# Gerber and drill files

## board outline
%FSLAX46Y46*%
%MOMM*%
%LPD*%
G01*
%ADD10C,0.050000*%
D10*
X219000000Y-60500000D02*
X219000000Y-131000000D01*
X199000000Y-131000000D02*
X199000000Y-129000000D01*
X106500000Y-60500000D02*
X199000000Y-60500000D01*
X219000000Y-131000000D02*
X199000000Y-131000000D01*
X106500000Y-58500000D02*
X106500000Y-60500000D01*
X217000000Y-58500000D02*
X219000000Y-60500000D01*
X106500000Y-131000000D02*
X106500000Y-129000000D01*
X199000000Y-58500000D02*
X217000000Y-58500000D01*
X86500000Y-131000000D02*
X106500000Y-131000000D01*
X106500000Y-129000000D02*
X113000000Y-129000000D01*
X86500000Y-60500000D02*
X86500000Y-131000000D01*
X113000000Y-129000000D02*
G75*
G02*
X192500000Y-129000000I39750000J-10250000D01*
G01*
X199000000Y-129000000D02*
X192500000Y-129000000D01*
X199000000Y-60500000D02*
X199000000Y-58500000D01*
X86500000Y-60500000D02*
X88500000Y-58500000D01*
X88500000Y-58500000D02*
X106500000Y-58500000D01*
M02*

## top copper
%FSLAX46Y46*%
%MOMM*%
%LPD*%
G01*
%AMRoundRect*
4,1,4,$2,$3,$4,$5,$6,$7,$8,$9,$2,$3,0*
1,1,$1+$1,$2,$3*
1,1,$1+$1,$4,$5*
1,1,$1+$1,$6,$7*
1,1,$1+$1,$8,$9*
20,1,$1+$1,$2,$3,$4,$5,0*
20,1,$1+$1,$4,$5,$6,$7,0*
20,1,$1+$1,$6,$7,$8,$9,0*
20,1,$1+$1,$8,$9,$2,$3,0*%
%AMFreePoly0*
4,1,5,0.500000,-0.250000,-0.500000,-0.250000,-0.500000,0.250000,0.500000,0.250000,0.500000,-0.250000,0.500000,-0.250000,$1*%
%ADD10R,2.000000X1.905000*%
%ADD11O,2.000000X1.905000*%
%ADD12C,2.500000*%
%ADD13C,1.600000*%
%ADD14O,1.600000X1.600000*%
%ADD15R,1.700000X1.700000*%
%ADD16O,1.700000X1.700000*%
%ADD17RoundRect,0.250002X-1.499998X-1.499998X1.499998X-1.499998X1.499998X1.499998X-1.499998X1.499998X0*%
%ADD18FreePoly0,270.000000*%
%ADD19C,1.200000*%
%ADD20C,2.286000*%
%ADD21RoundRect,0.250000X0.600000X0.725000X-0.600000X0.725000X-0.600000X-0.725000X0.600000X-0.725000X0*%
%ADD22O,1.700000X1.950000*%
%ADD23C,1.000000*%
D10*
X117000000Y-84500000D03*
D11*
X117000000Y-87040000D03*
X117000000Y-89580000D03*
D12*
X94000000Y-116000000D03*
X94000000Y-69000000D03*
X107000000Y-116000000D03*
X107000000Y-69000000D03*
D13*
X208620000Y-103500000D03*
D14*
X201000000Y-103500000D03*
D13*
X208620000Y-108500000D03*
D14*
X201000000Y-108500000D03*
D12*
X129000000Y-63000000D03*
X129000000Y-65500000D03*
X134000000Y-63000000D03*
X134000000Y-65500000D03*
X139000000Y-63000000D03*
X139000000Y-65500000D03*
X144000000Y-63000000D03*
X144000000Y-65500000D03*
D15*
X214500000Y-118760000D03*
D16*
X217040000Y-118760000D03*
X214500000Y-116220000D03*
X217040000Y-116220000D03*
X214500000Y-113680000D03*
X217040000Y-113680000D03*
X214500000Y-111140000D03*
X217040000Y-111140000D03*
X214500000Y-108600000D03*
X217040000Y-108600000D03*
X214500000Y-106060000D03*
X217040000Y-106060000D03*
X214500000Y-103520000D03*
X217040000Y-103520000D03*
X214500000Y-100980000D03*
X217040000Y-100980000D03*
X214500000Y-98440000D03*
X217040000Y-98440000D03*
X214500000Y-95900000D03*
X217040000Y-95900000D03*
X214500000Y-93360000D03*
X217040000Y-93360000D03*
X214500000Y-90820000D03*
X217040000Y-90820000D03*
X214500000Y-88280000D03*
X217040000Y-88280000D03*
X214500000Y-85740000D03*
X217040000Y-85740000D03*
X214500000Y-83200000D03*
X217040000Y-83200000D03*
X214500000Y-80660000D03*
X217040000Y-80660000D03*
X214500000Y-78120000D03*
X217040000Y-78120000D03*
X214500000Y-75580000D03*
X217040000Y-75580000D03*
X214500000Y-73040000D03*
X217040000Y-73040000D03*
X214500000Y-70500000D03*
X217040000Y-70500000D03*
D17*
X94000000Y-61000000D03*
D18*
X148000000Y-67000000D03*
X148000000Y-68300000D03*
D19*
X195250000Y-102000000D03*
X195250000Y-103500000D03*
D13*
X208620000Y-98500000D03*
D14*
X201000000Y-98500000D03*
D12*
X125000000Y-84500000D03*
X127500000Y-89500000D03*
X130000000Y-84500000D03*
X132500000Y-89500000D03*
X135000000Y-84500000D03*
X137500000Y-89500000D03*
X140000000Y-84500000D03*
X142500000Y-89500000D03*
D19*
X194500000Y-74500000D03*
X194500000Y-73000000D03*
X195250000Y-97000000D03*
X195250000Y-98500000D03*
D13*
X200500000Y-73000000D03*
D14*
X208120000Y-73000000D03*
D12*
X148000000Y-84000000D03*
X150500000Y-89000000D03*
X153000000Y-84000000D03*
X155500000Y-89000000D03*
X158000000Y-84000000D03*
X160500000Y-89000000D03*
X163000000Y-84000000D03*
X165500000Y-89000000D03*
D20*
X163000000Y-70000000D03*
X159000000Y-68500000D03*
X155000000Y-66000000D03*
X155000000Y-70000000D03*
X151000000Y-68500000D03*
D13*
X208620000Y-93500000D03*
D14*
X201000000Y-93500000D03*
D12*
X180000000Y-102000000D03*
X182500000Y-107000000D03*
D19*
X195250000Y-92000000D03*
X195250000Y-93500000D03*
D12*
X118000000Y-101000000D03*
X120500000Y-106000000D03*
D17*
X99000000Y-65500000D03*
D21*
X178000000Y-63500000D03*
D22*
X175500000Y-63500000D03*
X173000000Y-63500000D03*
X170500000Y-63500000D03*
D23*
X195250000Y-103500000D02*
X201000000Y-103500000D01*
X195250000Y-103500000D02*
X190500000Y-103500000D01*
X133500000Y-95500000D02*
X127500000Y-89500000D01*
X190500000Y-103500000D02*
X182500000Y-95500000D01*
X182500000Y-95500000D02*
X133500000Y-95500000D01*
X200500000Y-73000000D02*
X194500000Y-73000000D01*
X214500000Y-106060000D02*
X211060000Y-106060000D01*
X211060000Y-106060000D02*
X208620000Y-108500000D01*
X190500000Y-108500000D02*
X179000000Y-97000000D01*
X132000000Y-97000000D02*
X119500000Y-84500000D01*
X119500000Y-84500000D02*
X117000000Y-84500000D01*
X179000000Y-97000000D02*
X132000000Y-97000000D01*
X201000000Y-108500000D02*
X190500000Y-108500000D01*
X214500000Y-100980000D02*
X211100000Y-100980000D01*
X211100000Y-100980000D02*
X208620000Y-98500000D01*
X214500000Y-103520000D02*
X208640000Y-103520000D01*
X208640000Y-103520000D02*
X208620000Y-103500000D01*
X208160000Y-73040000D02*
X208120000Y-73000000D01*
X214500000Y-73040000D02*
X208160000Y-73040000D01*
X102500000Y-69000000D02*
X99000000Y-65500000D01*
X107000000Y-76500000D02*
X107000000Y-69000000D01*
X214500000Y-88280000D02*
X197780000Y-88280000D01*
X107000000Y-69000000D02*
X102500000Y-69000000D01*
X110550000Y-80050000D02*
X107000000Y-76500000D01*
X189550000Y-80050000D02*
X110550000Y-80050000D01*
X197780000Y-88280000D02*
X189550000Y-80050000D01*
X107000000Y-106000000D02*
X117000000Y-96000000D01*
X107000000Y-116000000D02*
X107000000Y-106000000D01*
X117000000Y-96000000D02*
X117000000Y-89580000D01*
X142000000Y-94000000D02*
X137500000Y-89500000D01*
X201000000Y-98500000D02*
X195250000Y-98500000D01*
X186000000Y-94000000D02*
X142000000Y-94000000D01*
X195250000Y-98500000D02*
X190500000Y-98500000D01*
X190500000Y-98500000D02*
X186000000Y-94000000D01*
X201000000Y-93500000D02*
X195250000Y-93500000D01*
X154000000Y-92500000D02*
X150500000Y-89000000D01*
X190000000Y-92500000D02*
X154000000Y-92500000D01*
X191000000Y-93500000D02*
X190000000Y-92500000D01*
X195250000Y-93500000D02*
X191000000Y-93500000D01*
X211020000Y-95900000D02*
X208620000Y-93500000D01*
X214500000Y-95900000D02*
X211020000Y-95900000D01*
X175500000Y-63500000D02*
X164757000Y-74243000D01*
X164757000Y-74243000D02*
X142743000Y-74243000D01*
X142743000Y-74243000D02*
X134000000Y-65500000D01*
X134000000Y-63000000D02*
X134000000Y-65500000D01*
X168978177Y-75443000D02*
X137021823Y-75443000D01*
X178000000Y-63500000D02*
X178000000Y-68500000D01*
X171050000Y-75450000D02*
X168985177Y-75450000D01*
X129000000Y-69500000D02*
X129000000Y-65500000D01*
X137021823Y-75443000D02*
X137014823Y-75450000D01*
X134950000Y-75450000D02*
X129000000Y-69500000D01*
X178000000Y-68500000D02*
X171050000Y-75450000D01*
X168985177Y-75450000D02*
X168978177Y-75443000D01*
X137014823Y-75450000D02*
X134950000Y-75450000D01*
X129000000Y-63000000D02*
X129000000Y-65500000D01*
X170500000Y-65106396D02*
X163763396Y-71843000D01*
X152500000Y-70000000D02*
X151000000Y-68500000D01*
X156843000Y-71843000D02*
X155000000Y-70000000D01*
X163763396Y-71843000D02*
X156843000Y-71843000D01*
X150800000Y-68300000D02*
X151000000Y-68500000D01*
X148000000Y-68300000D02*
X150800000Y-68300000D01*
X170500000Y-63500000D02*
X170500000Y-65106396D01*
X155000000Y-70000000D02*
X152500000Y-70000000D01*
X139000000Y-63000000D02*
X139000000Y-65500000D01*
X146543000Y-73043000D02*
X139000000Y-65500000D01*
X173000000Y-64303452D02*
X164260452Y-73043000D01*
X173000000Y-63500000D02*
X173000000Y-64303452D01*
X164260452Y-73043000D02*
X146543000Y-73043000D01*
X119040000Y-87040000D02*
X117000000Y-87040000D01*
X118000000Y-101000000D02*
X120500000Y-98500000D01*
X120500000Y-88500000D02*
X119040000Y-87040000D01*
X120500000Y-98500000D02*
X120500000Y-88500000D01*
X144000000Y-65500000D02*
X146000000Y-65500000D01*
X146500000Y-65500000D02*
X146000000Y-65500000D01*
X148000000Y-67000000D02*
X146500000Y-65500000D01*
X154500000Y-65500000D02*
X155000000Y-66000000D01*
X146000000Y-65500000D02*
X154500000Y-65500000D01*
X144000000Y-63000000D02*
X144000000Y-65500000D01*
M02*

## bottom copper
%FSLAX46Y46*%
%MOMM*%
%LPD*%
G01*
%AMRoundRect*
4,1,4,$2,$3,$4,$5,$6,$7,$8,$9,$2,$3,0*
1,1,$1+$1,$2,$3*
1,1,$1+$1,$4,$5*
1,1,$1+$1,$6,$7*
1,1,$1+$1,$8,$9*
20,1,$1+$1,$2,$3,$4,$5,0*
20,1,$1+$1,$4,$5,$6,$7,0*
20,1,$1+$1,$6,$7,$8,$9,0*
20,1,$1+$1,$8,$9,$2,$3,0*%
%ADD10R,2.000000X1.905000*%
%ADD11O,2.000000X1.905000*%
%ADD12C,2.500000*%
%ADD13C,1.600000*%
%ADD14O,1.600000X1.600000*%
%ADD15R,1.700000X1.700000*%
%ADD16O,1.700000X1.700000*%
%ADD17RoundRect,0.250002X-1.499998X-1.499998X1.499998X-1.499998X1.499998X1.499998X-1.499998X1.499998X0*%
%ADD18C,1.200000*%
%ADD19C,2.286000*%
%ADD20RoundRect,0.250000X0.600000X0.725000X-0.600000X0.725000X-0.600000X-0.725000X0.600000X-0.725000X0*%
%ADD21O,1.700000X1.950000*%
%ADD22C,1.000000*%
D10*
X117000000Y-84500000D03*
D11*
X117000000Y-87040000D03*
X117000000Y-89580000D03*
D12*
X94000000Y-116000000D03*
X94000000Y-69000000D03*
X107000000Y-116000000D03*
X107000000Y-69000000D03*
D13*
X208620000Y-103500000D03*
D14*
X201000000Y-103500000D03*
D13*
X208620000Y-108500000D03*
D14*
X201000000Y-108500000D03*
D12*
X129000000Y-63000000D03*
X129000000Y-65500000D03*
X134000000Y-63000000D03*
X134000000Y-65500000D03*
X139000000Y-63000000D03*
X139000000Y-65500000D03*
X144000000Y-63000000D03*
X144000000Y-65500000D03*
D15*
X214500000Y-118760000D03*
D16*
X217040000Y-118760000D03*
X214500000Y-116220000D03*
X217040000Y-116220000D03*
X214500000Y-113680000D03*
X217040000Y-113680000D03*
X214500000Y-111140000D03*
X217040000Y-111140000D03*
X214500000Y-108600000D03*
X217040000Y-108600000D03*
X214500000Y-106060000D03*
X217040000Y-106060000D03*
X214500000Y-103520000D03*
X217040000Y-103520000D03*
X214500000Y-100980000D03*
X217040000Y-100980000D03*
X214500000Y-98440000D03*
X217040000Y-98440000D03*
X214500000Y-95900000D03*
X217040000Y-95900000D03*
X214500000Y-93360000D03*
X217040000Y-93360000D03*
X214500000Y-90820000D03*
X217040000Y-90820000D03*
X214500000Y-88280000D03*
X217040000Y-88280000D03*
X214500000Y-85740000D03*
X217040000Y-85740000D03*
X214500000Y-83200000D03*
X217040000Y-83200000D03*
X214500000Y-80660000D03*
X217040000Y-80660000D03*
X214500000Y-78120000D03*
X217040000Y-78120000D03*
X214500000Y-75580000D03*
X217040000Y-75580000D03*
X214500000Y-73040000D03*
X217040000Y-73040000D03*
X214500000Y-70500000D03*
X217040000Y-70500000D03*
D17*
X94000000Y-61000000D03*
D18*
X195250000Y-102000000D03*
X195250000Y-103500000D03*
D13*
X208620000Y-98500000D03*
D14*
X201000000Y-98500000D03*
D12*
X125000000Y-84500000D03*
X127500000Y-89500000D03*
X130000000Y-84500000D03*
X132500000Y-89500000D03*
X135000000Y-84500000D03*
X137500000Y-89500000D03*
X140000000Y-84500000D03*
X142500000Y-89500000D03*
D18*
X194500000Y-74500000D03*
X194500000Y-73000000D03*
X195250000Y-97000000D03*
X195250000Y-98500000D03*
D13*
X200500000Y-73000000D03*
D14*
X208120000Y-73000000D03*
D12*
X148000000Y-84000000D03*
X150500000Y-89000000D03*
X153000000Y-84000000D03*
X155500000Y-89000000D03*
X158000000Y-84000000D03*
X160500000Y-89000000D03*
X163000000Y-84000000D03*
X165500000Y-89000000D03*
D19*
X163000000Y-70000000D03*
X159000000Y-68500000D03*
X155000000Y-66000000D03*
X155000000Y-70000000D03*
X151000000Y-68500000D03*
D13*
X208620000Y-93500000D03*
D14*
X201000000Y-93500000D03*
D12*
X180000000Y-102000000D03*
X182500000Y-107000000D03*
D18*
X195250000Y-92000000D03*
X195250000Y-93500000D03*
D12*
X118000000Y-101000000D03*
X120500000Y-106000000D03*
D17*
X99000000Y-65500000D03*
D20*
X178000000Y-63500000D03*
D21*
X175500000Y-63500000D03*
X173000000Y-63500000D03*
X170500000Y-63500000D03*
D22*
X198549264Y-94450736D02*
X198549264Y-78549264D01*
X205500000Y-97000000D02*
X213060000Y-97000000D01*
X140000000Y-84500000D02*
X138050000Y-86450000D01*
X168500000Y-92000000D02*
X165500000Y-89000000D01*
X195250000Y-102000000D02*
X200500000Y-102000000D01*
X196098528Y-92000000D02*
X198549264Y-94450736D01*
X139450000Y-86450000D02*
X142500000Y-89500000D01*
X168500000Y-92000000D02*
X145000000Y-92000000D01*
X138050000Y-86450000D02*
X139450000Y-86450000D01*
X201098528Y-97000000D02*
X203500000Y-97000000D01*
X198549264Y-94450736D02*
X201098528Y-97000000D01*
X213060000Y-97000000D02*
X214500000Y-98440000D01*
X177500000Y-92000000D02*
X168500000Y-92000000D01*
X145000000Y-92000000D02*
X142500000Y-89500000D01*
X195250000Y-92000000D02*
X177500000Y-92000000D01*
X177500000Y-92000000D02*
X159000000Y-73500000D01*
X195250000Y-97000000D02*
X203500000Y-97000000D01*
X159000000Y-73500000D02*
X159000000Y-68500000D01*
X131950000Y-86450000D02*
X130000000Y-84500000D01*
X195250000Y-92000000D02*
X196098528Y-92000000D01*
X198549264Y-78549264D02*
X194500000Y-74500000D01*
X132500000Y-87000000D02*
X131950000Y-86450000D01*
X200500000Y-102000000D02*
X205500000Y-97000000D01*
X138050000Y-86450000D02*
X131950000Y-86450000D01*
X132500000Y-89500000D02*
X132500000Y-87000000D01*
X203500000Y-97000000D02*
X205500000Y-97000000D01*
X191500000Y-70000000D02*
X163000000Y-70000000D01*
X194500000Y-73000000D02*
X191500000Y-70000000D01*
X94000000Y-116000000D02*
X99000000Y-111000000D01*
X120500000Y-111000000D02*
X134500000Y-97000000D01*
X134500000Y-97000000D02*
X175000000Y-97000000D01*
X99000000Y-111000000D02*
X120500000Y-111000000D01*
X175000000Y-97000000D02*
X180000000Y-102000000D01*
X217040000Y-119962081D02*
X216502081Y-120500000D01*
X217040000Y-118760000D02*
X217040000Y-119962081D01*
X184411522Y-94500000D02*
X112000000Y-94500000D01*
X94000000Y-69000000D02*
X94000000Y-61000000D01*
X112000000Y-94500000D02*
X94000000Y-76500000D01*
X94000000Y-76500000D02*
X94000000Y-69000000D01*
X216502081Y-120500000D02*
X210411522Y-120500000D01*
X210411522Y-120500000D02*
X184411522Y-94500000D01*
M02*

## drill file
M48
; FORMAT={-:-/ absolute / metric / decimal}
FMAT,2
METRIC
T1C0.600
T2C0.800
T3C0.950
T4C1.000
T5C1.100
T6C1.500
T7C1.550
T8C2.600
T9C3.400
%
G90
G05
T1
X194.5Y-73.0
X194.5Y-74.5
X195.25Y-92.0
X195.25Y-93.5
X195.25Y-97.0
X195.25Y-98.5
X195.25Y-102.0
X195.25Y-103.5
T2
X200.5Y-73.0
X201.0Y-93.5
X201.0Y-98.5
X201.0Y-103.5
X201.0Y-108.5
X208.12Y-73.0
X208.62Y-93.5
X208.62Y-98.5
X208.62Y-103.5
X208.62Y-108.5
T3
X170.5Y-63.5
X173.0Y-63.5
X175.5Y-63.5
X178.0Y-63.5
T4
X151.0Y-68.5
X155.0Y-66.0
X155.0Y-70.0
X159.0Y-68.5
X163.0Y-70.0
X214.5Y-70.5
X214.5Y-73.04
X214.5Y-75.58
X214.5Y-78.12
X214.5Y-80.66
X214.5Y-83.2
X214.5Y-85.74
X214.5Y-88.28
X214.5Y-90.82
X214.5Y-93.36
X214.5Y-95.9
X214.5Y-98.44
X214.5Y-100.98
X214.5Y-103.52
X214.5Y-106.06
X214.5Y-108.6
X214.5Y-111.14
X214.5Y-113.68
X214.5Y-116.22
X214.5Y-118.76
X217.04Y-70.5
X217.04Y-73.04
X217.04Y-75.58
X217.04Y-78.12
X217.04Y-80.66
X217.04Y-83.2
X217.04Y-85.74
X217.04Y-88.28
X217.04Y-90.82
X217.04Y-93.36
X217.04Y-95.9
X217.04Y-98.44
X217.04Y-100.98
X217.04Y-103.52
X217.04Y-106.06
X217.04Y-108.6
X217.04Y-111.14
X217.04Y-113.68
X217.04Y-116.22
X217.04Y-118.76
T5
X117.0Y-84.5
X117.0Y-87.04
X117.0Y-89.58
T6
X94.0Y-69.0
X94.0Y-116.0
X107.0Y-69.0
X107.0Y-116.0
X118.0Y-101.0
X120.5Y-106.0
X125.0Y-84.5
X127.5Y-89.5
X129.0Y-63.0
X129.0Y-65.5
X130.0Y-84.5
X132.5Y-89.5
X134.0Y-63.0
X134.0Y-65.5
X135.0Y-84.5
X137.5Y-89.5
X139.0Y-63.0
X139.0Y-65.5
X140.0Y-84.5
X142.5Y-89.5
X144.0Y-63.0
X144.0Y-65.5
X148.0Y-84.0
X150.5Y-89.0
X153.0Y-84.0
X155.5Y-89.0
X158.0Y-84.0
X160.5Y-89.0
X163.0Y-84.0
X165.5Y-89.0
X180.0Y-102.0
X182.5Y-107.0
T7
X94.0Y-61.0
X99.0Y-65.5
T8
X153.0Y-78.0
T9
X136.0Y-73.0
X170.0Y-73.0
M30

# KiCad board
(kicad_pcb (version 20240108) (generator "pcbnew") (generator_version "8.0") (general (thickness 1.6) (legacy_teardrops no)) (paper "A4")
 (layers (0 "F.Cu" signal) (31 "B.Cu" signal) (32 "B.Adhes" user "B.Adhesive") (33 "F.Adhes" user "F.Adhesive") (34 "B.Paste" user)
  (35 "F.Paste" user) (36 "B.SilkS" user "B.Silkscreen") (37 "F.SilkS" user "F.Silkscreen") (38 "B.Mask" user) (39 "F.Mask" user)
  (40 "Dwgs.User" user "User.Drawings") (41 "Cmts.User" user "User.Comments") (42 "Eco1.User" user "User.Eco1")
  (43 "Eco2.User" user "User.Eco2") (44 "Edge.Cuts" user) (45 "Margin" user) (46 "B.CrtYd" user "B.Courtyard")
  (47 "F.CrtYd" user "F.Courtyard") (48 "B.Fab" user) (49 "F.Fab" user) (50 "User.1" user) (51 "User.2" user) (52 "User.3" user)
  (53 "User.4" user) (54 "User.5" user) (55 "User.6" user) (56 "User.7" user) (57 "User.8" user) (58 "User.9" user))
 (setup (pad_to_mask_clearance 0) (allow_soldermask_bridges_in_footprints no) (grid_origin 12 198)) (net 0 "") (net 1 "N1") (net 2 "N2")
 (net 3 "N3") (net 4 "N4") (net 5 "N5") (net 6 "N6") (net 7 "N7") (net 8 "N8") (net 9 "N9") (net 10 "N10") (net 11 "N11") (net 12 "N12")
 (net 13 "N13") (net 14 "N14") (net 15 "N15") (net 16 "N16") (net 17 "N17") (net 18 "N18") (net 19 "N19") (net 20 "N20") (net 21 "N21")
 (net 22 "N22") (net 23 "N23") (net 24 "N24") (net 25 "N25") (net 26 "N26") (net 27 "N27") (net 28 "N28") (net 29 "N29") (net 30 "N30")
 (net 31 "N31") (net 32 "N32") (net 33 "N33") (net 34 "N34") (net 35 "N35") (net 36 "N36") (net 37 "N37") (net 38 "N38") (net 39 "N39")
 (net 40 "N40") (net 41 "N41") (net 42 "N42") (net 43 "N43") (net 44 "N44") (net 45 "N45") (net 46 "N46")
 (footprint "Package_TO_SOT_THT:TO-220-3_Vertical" (layer "F.Cu") (at 117 84.5 -90)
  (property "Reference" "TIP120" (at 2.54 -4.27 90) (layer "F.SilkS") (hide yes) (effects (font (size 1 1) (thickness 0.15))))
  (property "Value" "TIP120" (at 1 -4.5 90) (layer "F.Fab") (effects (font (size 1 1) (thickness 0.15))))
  (pad "1" thru_hole rect (at 0 0 270) (size 1.905 2) (drill 1.1) (layers "*.Cu" "*.Mask") (remove_unused_layers no) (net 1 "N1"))
  (pad "2" thru_hole oval (at 2.54 0 270) (size 1.905 2) (drill 1.1) (layers "*.Cu" "*.Mask") (remove_unused_layers no) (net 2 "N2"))
  (pad "3" thru_hole oval (at 5.08 0 270) (size 1.905 2) (drill 1.1) (layers "*.Cu" "*.Mask") (remove_unused_layers no) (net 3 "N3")))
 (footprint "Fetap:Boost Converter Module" (layer "F.Cu") (at 100.5 117.5)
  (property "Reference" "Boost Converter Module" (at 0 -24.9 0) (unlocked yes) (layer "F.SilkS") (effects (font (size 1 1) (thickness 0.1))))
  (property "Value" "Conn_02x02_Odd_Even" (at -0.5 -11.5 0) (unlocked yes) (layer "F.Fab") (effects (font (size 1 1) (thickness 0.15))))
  (pad "1" thru_hole circle (at -6.5 -1.5) (size 2.5 2.5) (drill 1.5) (layers "*.Cu" "*.Mask") (remove_unused_layers no) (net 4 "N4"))
  (pad "2" thru_hole circle (at -6.5 -48.5) (size 2.5 2.5) (drill 1.5) (layers "*.Cu" "*.Mask") (remove_unused_layers no) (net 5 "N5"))
  (pad "3" thru_hole circle (at 6.5 -1.5) (size 2.5 2.5) (drill 1.5) (layers "*.Cu" "*.Mask") (remove_unused_layers no) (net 3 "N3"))
  (pad "4" thru_hole circle (at 6.5 -48.5) (size 2.5 2.5) (drill 1.5) (layers "*.Cu" "*.Mask") (remove_unused_layers no) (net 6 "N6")))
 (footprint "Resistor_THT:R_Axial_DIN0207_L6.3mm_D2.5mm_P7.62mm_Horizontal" (layer "F.Cu") (at 208.62 103.5 180)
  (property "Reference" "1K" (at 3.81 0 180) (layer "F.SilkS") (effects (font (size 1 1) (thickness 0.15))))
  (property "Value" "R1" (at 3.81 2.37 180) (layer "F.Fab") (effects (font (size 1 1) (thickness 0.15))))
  (pad "1" thru_hole circle (at 0 0 180) (size 1.6 1.6) (drill 0.8) (layers "*.Cu" "*.Mask") (remove_unused_layers no) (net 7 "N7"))
  (pad "2" thru_hole oval (at 7.62 0 180) (size 1.6 1.6) (drill 0.8) (layers "*.Cu" "*.Mask") (remove_unused_layers no) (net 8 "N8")))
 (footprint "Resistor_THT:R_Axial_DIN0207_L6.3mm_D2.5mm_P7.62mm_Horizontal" (layer "F.Cu") (at 208.62 108.5 180)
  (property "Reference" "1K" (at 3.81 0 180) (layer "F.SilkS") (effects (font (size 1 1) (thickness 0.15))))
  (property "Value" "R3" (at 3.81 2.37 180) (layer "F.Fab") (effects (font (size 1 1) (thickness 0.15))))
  (pad "1" thru_hole circle (at 0 0 180) (size 1.6 1.6) (drill 0.8) (layers "*.Cu" "*.Mask") (remove_unused_layers no) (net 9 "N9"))
  (pad "2" thru_hole oval (at 7.62 0 180) (size 1.6 1.6) (drill 0.8) (layers "*.Cu" "*.Mask") (remove_unused_layers no) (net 1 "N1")))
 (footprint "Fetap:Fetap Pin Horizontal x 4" (layer "F.Cu") (at 129 65.5)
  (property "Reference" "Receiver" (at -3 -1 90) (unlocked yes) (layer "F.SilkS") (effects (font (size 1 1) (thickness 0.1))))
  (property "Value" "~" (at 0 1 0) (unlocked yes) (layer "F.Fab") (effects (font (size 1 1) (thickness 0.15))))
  (pad "1" thru_hole circle (at 0 -2.5) (size 2.5 2.5) (drill 1.5) (layers "*.Cu" "*.Mask") (remove_unused_layers no) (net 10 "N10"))
  (pad "1" thru_hole circle (at 0 0) (size 2.5 2.5) (drill 1.5) (layers "*.Cu" "*.Mask") (remove_unused_layers no) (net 10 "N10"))
  (pad "2" thru_hole circle (at 5 -2.5) (size 2.5 2.5) (drill 1.5) (layers "*.Cu" "*.Mask") (remove_unused_layers no) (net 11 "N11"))
  (pad "2" thru_hole circle (at 5 0) (size 2.5 2.5) (drill 1.5) (layers "*.Cu" "*.Mask") (remove_unused_layers no) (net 11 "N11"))
  (pad "3" thru_hole circle (at 10 -2.5) (size 2.5 2.5) (drill 1.5) (layers "*.Cu" "*.Mask") (remove_unused_layers no) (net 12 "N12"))
  (pad "3" thru_hole circle (at 10 0) (size 2.5 2.5) (drill 1.5) (layers "*.Cu" "*.Mask") (remove_unused_layers no) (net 12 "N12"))
  (pad "4" thru_hole circle (at 15 -2.5) (size 2.5 2.5) (drill 1.5) (layers "*.Cu" "*.Mask") (remove_unused_layers no) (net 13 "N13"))
  (pad "4" thru_hole circle (at 15 0) (size 2.5 2.5) (drill 1.5) (layers "*.Cu" "*.Mask") (remove_unused_layers no) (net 13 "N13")))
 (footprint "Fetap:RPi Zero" (layer "F.Cu") (at 214.5 118.76 180)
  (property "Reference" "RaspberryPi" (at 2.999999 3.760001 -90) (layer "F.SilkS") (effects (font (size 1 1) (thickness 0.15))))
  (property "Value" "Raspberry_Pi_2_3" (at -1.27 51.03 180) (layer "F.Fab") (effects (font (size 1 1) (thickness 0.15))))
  (pad "1" thru_hole rect (at 0 0 180) (size 1.7 1.7) (drill 1) (layers "*.Cu" "*.Mask") (remove_unused_layers no) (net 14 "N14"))
  (pad "2" thru_hole oval (at -2.54 0 180) (size 1.7 1.7) (drill 1) (layers "*.Cu" "*.Mask") (remove_unused_layers no) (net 5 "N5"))
  (pad "3" thru_hole oval (at 0 2.54 180) (size 1.7 1.7) (drill 1) (layers "*.Cu" "*.Mask") (remove_unused_layers no) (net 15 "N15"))
  (pad "4" thru_hole oval (at -2.54 2.54 180) (size 1.7 1.7) (drill 1) (layers "*.Cu" "*.Mask") (remove_unused_layers no) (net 5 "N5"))
  (pad "5" thru_hole oval (at 0 5.08 180) (size 1.7 1.7) (drill 1) (layers "*.Cu" "*.Mask") (remove_unused_layers no) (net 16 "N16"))
  (pad "6" thru_hole oval (at -2.54 5.08 180) (size 1.7 1.7) (drill 1) (layers "*.Cu" "*.Mask") (remove_unused_layers no) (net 6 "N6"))
  (pad "7" thru_hole oval (at 0 7.62 180) (size 1.7 1.7) (drill 1) (layers "*.Cu" "*.Mask") (remove_unused_layers no) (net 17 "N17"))
  (pad "8" thru_hole oval (at -2.54 7.62 180) (size 1.7 1.7) (drill 1) (layers "*.Cu" "*.Mask") (remove_unused_layers no) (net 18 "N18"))
  (pad "9" thru_hole oval (at 0 10.16 180) (size 1.7 1.7) (drill 1) (layers "*.Cu" "*.Mask") (remove_unused_layers no) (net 6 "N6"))
  (pad "10" thru_hole oval (at -2.54 10.16 180) (size 1.7 1.7) (drill 1) (layers "*.Cu" "*.Mask") (remove_unused_layers no) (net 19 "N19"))
  (pad "11" thru_hole oval (at 0 12.7 180) (size 1.7 1.7) (drill 1) (layers "*.Cu" "*.Mask") (remove_unused_layers no) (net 9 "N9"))
  (pad "12" thru_hole oval (at -2.54 12.7 180) (size 1.7 1.7) (drill 1) (layers "*.Cu" "*.Mask") (remove_unused_layers no) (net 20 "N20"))
  (pad "13" thru_hole oval (at 0 15.24 180) (size 1.7 1.7) (drill 1) (layers "*.Cu" "*.Mask") (remove_unused_layers no) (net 7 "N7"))
  (pad "14" thru_hole oval (at -2.54 15.24 180) (size 1.7 1.7) (drill 1) (layers "*.Cu" "*.Mask") (remove_unused_layers no) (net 6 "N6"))
  (pad "15" thru_hole oval (at 0 17.78 180) (size 1.7 1.7) (drill 1) (layers "*.Cu" "*.Mask") (remove_unused_layers no) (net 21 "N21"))
  (pad "16" thru_hole oval (at -2.54 17.78 180) (size 1.7 1.7) (drill 1) (layers "*.Cu" "*.Mask") (remove_unused_layers no) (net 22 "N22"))
  (pad "17" thru_hole oval (at 0 20.32 180) (size 1.7 1.7) (drill 1) (layers "*.Cu" "*.Mask") (remove_unused_layers no) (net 14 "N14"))
  (pad "18" thru_hole oval (at -2.54 20.32 180) (size 1.7 1.7) (drill 1) (layers "*.Cu" "*.Mask") (remove_unused_layers no) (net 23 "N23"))
  (pad "19" thru_hole oval (at 0 22.86 180) (size 1.7 1.7) (drill 1) (layers "*.Cu" "*.Mask") (remove_unused_layers no) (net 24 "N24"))
  (pad "20" thru_hole oval (at -2.54 22.86 180) (size 1.7 1.7) (drill 1) (layers "*.Cu" "*.Mask") (remove_unused_layers no) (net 6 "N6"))
  (pad "21" thru_hole oval (at 0 25.4 180) (size 1.7 1.7) (drill 1) (layers "*.Cu" "*.Mask") (remove_unused_layers no) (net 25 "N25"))
  (pad "22" thru_hole oval (at -2.54 25.4 180) (size 1.7 1.7) (drill 1) (layers "*.Cu" "*.Mask") (remove_unused_layers no) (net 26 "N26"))
  (pad "23" thru_hole oval (at 0 27.94 180) (size 1.7 1.7) (drill 1) (layers "*.Cu" "*.Mask") (remove_unused_layers no) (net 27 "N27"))
  (pad "24" thru_hole oval (at -2.54 27.94 180) (size 1.7 1.7) (drill 1) (layers "*.Cu" "*.Mask") (remove_unused_layers no) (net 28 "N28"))
  (pad "25" thru_hole oval (at 0 30.48 180) (size 1.7 1.7) (drill 1) (layers "*.Cu" "*.Mask") (remove_unused_layers no) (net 6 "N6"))
  (pad "26" thru_hole oval (at -2.54 30.48 180) (size 1.7 1.7) (drill 1) (layers "*.Cu" "*.Mask") (remove_unused_layers no) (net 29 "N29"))
  (pad "27" thru_hole oval (at 0 33.02 180) (size 1.7 1.7) (drill 1) (layers "*.Cu" "*.Mask") (remove_unused_layers no) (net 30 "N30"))
  (pad "28" thru_hole oval (at -2.54 33.02 180) (size 1.7 1.7) (drill 1) (layers "*.Cu" "*.Mask") (remove_unused_layers no) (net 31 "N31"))
  (pad "29" thru_hole oval (at 0 35.56 180) (size 1.7 1.7) (drill 1) (layers "*.Cu" "*.Mask") (remove_unused_layers no) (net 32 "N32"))
  (pad "30" thru_hole oval (at -2.54 35.56 180) (size 1.7 1.7) (drill 1) (layers "*.Cu" "*.Mask") (remove_unused_layers no) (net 6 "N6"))
  (pad "31" thru_hole oval (at 0 38.1 180) (size 1.7 1.7) (drill 1) (layers "*.Cu" "*.Mask") (remove_unused_layers no) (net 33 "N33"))
  (pad "32" thru_hole oval (at -2.54 38.1 180) (size 1.7 1.7) (drill 1) (layers "*.Cu" "*.Mask") (remove_unused_layers no) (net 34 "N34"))
  (pad "33" thru_hole oval (at 0 40.64 180) (size 1.7 1.7) (drill 1) (layers "*.Cu" "*.Mask") (remove_unused_layers no) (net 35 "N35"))
  (pad "34" thru_hole oval (at -2.54 40.64 180) (size 1.7 1.7) (drill 1) (layers "*.Cu" "*.Mask") (remove_unused_layers no) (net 6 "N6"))
  (pad "35" thru_hole oval (at 0 43.18 180) (size 1.7 1.7) (drill 1) (layers "*.Cu" "*.Mask") (remove_unused_layers no) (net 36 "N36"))
  (pad "36" thru_hole oval (at -2.54 43.18 180) (size 1.7 1.7) (drill 1) (layers "*.Cu" "*.Mask") (remove_unused_layers no) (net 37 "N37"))
  (pad "37" thru_hole oval (at 0 45.72 180) (size 1.7 1.7) (drill 1) (layers "*.Cu" "*.Mask") (remove_unused_layers no) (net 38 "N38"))
  (pad "38" thru_hole oval (at -2.54 45.72 180) (size 1.7 1.7) (drill 1) (layers "*.Cu" "*.Mask") (remove_unused_layers no) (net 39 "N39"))
  (pad "39" thru_hole oval (at 0 48.26 180) (size 1.7 1.7) (drill 1) (layers "*.Cu" "*.Mask") (remove_unused_layers no) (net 6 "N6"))
  (pad "40" thru_hole oval (at -2.54 48.26 180) (size 1.7 1.7) (drill 1) (layers "*.Cu" "*.Mask") (remove_unused_layers no) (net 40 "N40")))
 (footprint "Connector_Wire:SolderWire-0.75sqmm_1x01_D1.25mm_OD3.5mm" (layer "F.Cu") (at 94 61)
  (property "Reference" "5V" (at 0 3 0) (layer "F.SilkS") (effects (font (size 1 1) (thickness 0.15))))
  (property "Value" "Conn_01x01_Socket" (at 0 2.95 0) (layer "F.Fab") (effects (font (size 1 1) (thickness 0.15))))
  (pad "1" thru_hole roundrect (at 0 0) (size 3.5 3.5) (drill 1.55) (layers "*.Cu" "*.Mask") (remove_unused_layers no)
   (roundrect_rratio 0.071429) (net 5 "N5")))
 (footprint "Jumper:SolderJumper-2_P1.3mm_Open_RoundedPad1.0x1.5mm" (layer "F.Cu") (at 148 67.65 -90)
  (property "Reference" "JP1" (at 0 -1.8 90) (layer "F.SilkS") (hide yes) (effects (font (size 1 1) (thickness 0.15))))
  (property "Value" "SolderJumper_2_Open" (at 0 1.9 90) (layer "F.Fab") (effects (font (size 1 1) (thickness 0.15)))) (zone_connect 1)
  (pad "1" smd custom (at -0.65 0 270) (size 1 0.5) (layers "F.Cu" "F.Mask") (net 13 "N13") (zone_connect 2) (thermal_bridge_angle 45)
   (options (clearance outline) (anchor rect)) (primitives))
  (pad "2" smd custom (at 0.65 0 270) (size 1 0.5) (layers "F.Cu" "F.Mask") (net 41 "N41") (zone_connect 2) (thermal_bridge_angle 45)
   (options (clearance outline) (anchor rect)) (primitives)))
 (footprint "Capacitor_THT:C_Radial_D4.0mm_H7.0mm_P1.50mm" (layer "F.Cu") (at 195.25 102 -90)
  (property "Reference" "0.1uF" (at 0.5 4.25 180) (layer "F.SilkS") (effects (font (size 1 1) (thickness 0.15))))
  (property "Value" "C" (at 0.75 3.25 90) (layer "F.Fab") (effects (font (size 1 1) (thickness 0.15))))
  (pad "1" thru_hole circle (at 0 0 270) (size 1.2 1.2) (drill 0.6) (layers "*.Cu" "*.Mask") (remove_unused_layers no) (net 14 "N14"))
  (pad "2" thru_hole circle (at 1.5 0 270) (size 1.2 1.2) (drill 0.6) (layers "*.Cu" "*.Mask") (remove_unused_layers no) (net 8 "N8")))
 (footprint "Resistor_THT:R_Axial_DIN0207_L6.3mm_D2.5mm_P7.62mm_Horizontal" (layer "F.Cu") (at 208.62 98.5 180)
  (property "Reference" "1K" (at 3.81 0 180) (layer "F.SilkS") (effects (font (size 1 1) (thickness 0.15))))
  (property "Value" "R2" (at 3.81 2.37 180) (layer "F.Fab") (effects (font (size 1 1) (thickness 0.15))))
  (pad "1" thru_hole circle (at 0 0 180) (size 1.6 1.6) (drill 0.8) (layers "*.Cu" "*.Mask") (remove_unused_layers no) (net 21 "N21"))
  (pad "2" thru_hole oval (at 7.62 0 180) (size 1.6 1.6) (drill 0.8) (layers "*.Cu" "*.Mask") (remove_unused_layers no) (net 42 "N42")))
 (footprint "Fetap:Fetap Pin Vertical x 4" (layer "F.Cu") (at 127.5 89.5)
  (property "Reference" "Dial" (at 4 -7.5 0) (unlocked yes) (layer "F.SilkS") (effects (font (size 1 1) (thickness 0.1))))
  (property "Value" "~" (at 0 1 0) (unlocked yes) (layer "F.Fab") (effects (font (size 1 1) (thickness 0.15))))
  (pad "1" thru_hole circle (at -2.5 -5) (size 2.5 2.5) (drill 1.5) (layers "*.Cu" "*.Mask") (remove_unused_layers no) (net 8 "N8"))
  (pad "1" thru_hole circle (at 0 0) (size 2.5 2.5) (drill 1.5) (layers "*.Cu" "*.Mask") (remove_unused_layers no) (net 8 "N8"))
  (pad "2" thru_hole circle (at 2.5 -5) (size 2.5 2.5) (drill 1.5) (layers "*.Cu" "*.Mask") (remove_unused_layers no) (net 14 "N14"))
  (pad "2" thru_hole circle (at 5 0) (size 2.5 2.5) (drill 1.5) (layers "*.Cu" "*.Mask") (remove_unused_layers no) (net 14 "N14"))
  (pad "3" thru_hole circle (at 7.5 -5) (size 2.5 2.5) (drill 1.5) (layers "*.Cu" "*.Mask") (remove_unused_layers no) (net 42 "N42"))
  (pad "3" thru_hole circle (at 10 0) (size 2.5 2.5) (drill 1.5) (layers "*.Cu" "*.Mask") (remove_unused_layers no) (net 42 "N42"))
  (pad "4" thru_hole circle (at 12.5 -5) (size 2.5 2.5) (drill 1.5) (layers "*.Cu" "*.Mask") (remove_unused_layers no) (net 14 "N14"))
  (pad "4" thru_hole circle (at 15 0) (size 2.5 2.5) (drill 1.5) (layers "*.Cu" "*.Mask") (remove_unused_layers no) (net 14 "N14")))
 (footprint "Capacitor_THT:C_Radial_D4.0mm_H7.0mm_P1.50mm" (layer "F.Cu") (at 194.5 74.5 90)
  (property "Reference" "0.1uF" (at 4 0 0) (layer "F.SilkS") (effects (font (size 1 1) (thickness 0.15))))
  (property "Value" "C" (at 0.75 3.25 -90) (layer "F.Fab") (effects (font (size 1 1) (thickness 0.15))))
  (pad "1" thru_hole circle (at 0 0 90) (size 1.2 1.2) (drill 0.6) (layers "*.Cu" "*.Mask") (remove_unused_layers no) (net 14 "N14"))
  (pad "2" thru_hole circle (at 1.5 0 90) (size 1.2 1.2) (drill 0.6) (layers "*.Cu" "*.Mask") (remove_unused_layers no) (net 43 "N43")))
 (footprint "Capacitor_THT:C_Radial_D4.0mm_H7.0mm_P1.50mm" (layer "F.Cu") (at 195.25 97 -90)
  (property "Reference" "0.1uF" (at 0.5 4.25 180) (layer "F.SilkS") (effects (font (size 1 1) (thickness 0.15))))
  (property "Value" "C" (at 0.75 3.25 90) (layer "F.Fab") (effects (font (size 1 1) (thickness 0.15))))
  (pad "1" thru_hole circle (at 0 0 270) (size 1.2 1.2) (drill 0.6) (layers "*.Cu" "*.Mask") (remove_unused_layers no) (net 14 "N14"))
  (pad "2" thru_hole circle (at 1.5 0 270) (size 1.2 1.2) (drill 0.6) (layers "*.Cu" "*.Mask") (remove_unused_layers no) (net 42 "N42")))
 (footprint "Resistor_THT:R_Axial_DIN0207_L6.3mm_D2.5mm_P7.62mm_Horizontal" (layer "F.Cu") (at 200.5 73)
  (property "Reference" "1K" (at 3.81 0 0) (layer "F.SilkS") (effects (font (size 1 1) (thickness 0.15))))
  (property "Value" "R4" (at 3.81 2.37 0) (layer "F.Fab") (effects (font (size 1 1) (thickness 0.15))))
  (pad "1" thru_hole circle (at 0 0) (size 1.6 1.6) (drill 0.8) (layers "*.Cu" "*.Mask") (remove_unused_layers no) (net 43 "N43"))
  (pad "2" thru_hole oval (at 7.62 0) (size 1.6 1.6) (drill 0.8) (layers "*.Cu" "*.Mask") (remove_unused_layers no) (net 38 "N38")))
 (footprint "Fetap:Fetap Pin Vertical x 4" (layer "F.Cu") (at 150.5 89)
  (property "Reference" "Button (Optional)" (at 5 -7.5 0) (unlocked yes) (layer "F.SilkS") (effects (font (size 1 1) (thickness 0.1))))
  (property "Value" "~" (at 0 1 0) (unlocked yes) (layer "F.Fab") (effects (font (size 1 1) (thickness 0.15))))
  (pad "1" thru_hole circle (at -2.5 -5) (size 2.5 2.5) (drill 1.5) (layers "*.Cu" "*.Mask") (remove_unused_layers no) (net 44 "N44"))
  (pad "1" thru_hole circle (at 0 0) (size 2.5 2.5) (drill 1.5) (layers "*.Cu" "*.Mask") (remove_unused_layers no) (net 44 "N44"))
  (pad "2" thru_hole circle (at 2.5 -5) (size 2.5 2.5) (drill 1.5) (layers "*.Cu" "*.Mask") (remove_unused_layers no) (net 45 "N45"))
  (pad "2" thru_hole circle (at 5 0) (size 2.5 2.5) (drill 1.5) (layers "*.Cu" "*.Mask") (remove_unused_layers no) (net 45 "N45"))
  (pad "3" thru_hole circle (at 7.5 -5) (size 2.5 2.5) (drill 1.5) (layers "*.Cu" "*.Mask") (remove_unused_layers no) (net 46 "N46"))
  (pad "3" thru_hole circle (at 10 0) (size 2.5 2.5) (drill 1.5) (layers "*.Cu" "*.Mask") (remove_unused_layers no) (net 46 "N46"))
  (pad "4" thru_hole circle (at 12.5 -5) (size 2.5 2.5) (drill 1.5) (layers "*.Cu" "*.Mask") (remove_unused_layers no) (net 14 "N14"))
  (pad "4" thru_hole circle (at 15 0) (size 2.5 2.5) (drill 1.5) (layers "*.Cu" "*.Mask") (remove_unused_layers no) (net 14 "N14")))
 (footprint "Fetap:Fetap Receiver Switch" (layer "F.Cu") (at 153 70 180)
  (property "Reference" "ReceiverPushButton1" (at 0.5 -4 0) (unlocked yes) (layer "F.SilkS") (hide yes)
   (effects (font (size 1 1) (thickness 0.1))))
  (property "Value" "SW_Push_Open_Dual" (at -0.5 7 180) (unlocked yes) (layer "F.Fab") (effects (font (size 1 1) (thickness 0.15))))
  (pad "" np_thru_hole circle (at -17 -3 180) (size 3.4 3.4) (drill 3.4) (layers "*.Mask"))
  (pad "" np_thru_hole circle (at 0 -8 180) (size 2.6 2.6) (drill 2.6) (layers "F&B.Cu" "*.Mask"))
  (pad "" np_thru_hole circle (at 17 -3 180) (size 3.4 3.4) (drill 3.4) (layers "*.Mask"))
  (pad "1" thru_hole circle (at -10 0 180) (size 2.286 2.286) (drill 1) (layers "*.Cu" "*.Mask") (remove_unused_layers no) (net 43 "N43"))
  (pad "2" thru_hole circle (at -6 1.5 180) (size 2.286 2.286) (drill 1) (layers "*.Cu" "*.Mask") (remove_unused_layers no) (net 14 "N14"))
  (pad "3" thru_hole circle (at -2 4 180) (size 2.286 2.286) (drill 1) (layers "*.Cu" "*.Mask") (remove_unused_layers no) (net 13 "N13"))
  (pad "4" thru_hole circle (at -2 0 180) (size 2.286 2.286) (drill 1) (layers "*.Cu" "*.Mask") (remove_unused_layers no) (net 41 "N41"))
  (pad "4" thru_hole circle (at 2 1.5 180) (size 2.286 2.286) (drill 1) (layers "*.Cu" "*.Mask") (remove_unused_layers no) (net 41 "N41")))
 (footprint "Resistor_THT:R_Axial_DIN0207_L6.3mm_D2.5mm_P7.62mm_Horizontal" (layer "F.Cu") (at 208.62 93.5 180)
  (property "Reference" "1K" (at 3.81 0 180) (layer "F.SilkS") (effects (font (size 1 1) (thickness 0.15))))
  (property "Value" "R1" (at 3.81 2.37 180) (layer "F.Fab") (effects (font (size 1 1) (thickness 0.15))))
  (pad "1" thru_hole circle (at 0 0 180) (size 1.6 1.6) (drill 0.8) (layers "*.Cu" "*.Mask") (remove_unused_layers no) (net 24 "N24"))
  (pad "2" thru_hole oval (at 7.62 0 180) (size 1.6 1.6) (drill 0.8) (layers "*.Cu" "*.Mask") (remove_unused_layers no) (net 44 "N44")))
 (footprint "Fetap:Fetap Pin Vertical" (layer "F.Cu") (at 182.5 107)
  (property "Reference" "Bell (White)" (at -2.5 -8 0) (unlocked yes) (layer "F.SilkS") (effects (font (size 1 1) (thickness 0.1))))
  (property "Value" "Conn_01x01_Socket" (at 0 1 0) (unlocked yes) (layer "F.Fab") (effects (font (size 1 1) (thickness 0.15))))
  (pad "1" thru_hole circle (at -2.5 -5) (size 2.5 2.5) (drill 1.5) (layers "*.Cu" "*.Mask") (remove_unused_layers no) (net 4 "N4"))
  (pad "1" thru_hole circle (at 0 0) (size 2.5 2.5) (drill 1.5) (layers "*.Cu" "*.Mask") (remove_unused_layers no) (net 4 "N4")))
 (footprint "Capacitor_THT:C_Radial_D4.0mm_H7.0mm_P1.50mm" (layer "F.Cu") (at 195.25 92 -90)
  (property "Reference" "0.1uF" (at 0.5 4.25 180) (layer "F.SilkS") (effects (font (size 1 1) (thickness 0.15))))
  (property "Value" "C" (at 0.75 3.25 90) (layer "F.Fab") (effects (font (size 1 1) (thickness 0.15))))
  (pad "1" thru_hole circle (at 0 0 270) (size 1.2 1.2) (drill 0.6) (layers "*.Cu" "*.Mask") (remove_unused_layers no) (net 14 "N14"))
  (pad "2" thru_hole circle (at 1.5 0 270) (size 1.2 1.2) (drill 0.6) (layers "*.Cu" "*.Mask") (remove_unused_layers no) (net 44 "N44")))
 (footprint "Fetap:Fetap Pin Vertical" (layer "F.Cu") (at 120.5 106)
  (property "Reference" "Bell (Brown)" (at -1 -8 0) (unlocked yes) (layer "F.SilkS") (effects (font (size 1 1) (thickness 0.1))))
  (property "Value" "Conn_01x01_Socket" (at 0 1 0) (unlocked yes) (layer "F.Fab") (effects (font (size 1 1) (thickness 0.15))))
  (pad "1" thru_hole circle (at -2.5 -5) (size 2.5 2.5) (drill 1.5) (layers "*.Cu" "*.Mask") (remove_unused_layers no) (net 2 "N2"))
  (pad "1" thru_hole circle (at 0 0) (size 2.5 2.5) (drill 1.5) (layers "*.Cu" "*.Mask") (remove_unused_layers no) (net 2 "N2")))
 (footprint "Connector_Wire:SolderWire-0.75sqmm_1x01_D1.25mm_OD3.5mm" (layer "F.Cu") (at 99 65.5)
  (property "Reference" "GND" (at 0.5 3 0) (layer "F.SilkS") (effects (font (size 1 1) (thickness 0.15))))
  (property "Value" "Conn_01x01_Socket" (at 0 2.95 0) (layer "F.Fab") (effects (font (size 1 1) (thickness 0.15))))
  (pad "1" thru_hole roundrect (at 0 0) (size 3.5 3.5) (drill 1.55) (layers "*.Cu" "*.Mask") (remove_unused_layers no)
   (roundrect_rratio 0.071429) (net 6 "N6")))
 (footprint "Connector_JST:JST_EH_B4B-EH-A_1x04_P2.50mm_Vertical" (layer "F.Cu") (at 178 63.5 180)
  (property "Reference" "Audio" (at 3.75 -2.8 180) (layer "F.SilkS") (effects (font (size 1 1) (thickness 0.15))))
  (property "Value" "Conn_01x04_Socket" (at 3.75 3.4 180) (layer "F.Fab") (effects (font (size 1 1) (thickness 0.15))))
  (pad "1" thru_hole roundrect (at 0 0 180) (size 1.7 1.95) (drill 0.95) (layers "*.Cu" "*.Mask") (remove_unused_layers no)
   (roundrect_rratio 0.147059) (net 10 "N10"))
  (pad "2" thru_hole oval (at 2.5 0 180) (size 1.7 1.95) (drill 0.95) (layers "*.Cu" "*.Mask") (remove_unused_layers no) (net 11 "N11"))
  (pad "3" thru_hole oval (at 5 0 180) (size 1.7 1.95) (drill 0.95) (layers "*.Cu" "*.Mask") (remove_unused_layers no) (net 12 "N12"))
  (pad "4" thru_hole oval (at 7.5 0 180) (size 1.7 1.95) (drill 0.95) (layers "*.Cu" "*.Mask") (remove_unused_layers no) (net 41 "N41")))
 (gr_line (start 219 60.5) (end 219 131) (stroke (width 0.05) (type default)) (layer "Edge.Cuts"))
 (gr_line (start 199 131) (end 199 129) (stroke (width 0.05) (type default)) (layer "Edge.Cuts"))
 (gr_line (start 106.5 60.5) (end 199 60.5) (stroke (width 0.05) (type default)) (layer "Edge.Cuts"))
 (gr_line (start 219 131) (end 199 131) (stroke (width 0.05) (type default)) (layer "Edge.Cuts"))
 (gr_line (start 106.5 58.5) (end 106.5 60.5) (stroke (width 0.05) (type default)) (layer "Edge.Cuts"))
 (gr_line (start 217 58.5) (end 219 60.5) (stroke (width 0.05) (type default)) (layer "Edge.Cuts"))
 (gr_line (start 106.5 131) (end 106.5 129) (stroke (width 0.05) (type default)) (layer "Edge.Cuts"))
 (gr_line (start 199 58.5) (end 217 58.5) (stroke (width 0.05) (type default)) (layer "Edge.Cuts"))
 (gr_line (start 86.5 131) (end 106.5 131) (stroke (width 0.05) (type default)) (layer "Edge.Cuts"))
 (gr_line (start 106.5 129) (end 113 129) (stroke (width 0.05) (type default)) (layer "Edge.Cuts"))
 (gr_line (start 86.5 60.5) (end 86.5 131) (stroke (width 0.05) (type default)) (layer "Edge.Cuts"))
 (gr_arc (start 113 129) (mid 152.75 98.199726) (end 192.5 129) (stroke (width 0.05) (type default)) (layer "Edge.Cuts"))
 (gr_line (start 199 129) (end 192.5 129) (stroke (width 0.05) (type default)) (layer "Edge.Cuts"))
 (gr_line (start 199 60.5) (end 199 58.5) (stroke (width 0.05) (type default)) (layer "Edge.Cuts"))
 (gr_line (start 86.5 60.5) (end 88.5 58.5) (stroke (width 0.05) (type default)) (layer "Edge.Cuts"))
 (gr_line (start 88.5 58.5) (end 106.5 58.5) (stroke (width 0.05) (type default)) (layer "Edge.Cuts"))
 (segment (start 198.549264 94.450736) (end 198.549264 78.549264) (width 1) (layer "B.Cu") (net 14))
 (segment (start 205.5 97) (end 213.06 97) (width 1) (layer "B.Cu") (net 14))
 (segment (start 140 84.5) (end 138.05 86.45) (width 1) (layer "B.Cu") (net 14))
 (segment (start 168.5 92) (end 165.5 89) (width 1) (layer "B.Cu") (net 14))
 (segment (start 195.25 102) (end 200.5 102) (width 1) (layer "B.Cu") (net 14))
 (segment (start 196.098528 92) (end 198.549264 94.450736) (width 1) (layer "B.Cu") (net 14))
 (segment (start 139.45 86.45) (end 142.5 89.5) (width 1) (layer "B.Cu") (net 14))
 (segment (start 168.5 92) (end 145 92) (width 1) (layer "B.Cu") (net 14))
 (segment (start 138.05 86.45) (end 139.45 86.45) (width 1) (layer "B.Cu") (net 14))
 (segment (start 201.098528 97) (end 203.5 97) (width 1) (layer "B.Cu") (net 14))
 (segment (start 198.549264 94.450736) (end 201.098528 97) (width 1) (layer "B.Cu") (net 14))
 (segment (start 213.06 97) (end 214.5 98.44) (width 1) (layer "B.Cu") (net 14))
 (segment (start 177.5 92) (end 168.5 92) (width 1) (layer "B.Cu") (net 14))
 (segment (start 145 92) (end 142.5 89.5) (width 1) (layer "B.Cu") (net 14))
 (segment (start 195.25 92) (end 177.5 92) (width 1) (layer "B.Cu") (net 14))
 (segment (start 177.5 92) (end 159 73.5) (width 1) (layer "B.Cu") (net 14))
 (segment (start 195.25 97) (end 203.5 97) (width 1) (layer "B.Cu") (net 14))
 (segment (start 159 73.5) (end 159 68.5) (width 1) (layer "B.Cu") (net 14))
 (segment (start 131.95 86.45) (end 130 84.5) (width 1) (layer "B.Cu") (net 14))
 (segment (start 195.25 92) (end 196.098528 92) (width 1) (layer "B.Cu") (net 14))
 (segment (start 198.549264 78.549264) (end 194.5 74.5) (width 1) (layer "B.Cu") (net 14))
 (segment (start 132.5 87) (end 131.95 86.45) (width 1) (layer "B.Cu") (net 14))
 (segment (start 200.5 102) (end 205.5 97) (width 1) (layer "B.Cu") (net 14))
 (segment (start 138.05 86.45) (end 131.95 86.45) (width 1) (layer "B.Cu") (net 14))
 (segment (start 132.5 89.5) (end 132.5 87) (width 1) (layer "B.Cu") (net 14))
 (segment (start 203.5 97) (end 205.5 97) (width 1) (layer "B.Cu") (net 14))
 (segment (start 195.25 103.5) (end 201 103.5) (width 1) (layer "F.Cu") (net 8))
 (segment (start 195.25 103.5) (end 190.5 103.5) (width 1) (layer "F.Cu") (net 8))
 (segment (start 133.5 95.5) (end 127.5 89.5) (width 1) (layer "F.Cu") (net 8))
 (segment (start 190.5 103.5) (end 182.5 95.5) (width 1) (layer "F.Cu") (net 8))
 (segment (start 182.5 95.5) (end 133.5 95.5) (width 1) (layer "F.Cu") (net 8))
 (segment (start 200.5 73) (end 194.5 73) (width 1) (layer "F.Cu") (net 43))
 (segment (start 191.5 70) (end 163 70) (width 1) (layer "B.Cu") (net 43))
 (segment (start 194.5 73) (end 191.5 70) (width 1) (layer "B.Cu") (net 43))
 (segment (start 214.5 106.06) (end 211.06 106.06) (width 1) (layer "F.Cu") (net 9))
 (segment (start 211.06 106.06) (end 208.62 108.5) (width 1) (layer "F.Cu") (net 9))
 (segment (start 190.5 108.5) (end 179 97) (width 1) (layer "F.Cu") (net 1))
 (segment (start 132 97) (end 119.5 84.5) (width 1) (layer "F.Cu") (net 1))
 (segment (start 119.5 84.5) (end 117 84.5) (width 1) (layer "F.Cu") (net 1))
 (segment (start 179 97) (end 132 97) (width 1) (layer "F.Cu") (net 1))
 (segment (start 201 108.5) (end 190.5 108.5) (width 1) (layer "F.Cu") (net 1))
 (segment (start 214.5 100.98) (end 211.1 100.98) (width 1) (layer "F.Cu") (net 21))
 (segment (start 211.1 100.98) (end 208.62 98.5) (width 1) (layer "F.Cu") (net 21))
 (segment (start 214.5 103.52) (end 208.64 103.52) (width 1) (layer "F.Cu") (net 7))
 (segment (start 208.64 103.52) (end 208.62 103.5) (width 1) (layer "F.Cu") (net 7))
 (segment (start 208.16 73.04) (end 208.12 73) (width 1) (layer "F.Cu") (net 38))
 (segment (start 214.5 73.04) (end 208.16 73.04) (width 1) (layer "F.Cu") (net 38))
 (segment (start 102.5 69) (end 99 65.5) (width 1) (layer "F.Cu") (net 6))
 (segment (start 107 76.5) (end 107 69) (width 1) (layer "F.Cu") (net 6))
 (segment (start 214.5 88.28) (end 197.78 88.28) (width 1) (layer "F.Cu") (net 6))
 (segment (start 107 69) (end 102.5 69) (width 1) (layer "F.Cu") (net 6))
 (segment (start 110.55 80.05) (end 107 76.5) (width 1) (layer "F.Cu") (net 6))
 (segment (start 189.55 80.05) (end 110.55 80.05) (width 1) (layer "F.Cu") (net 6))
 (segment (start 197.78 88.28) (end 189.55 80.05) (width 1) (layer "F.Cu") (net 6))
 (segment (start 107 106) (end 117 96) (width 1) (layer "F.Cu") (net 3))
 (segment (start 107 116) (end 107 106) (width 1) (layer "F.Cu") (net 3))
 (segment (start 117 96) (end 117 89.58) (width 1) (layer "F.Cu") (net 3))
 (segment (start 142 94) (end 137.5 89.5) (width 1) (layer "F.Cu") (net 42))
 (segment (start 201 98.5) (end 195.25 98.5) (width 1) (layer "F.Cu") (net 42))
 (segment (start 186 94) (end 142 94) (width 1) (layer "F.Cu") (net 42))
 (segment (start 195.25 98.5) (end 190.5 98.5) (width 1) (layer "F.Cu") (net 42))
 (segment (start 190.5 98.5) (end 186 94) (width 1) (layer "F.Cu") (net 42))
 (segment (start 201 93.5) (end 195.25 93.5) (width 1) (layer "F.Cu") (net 44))
 (segment (start 154 92.5) (end 150.5 89) (width 1) (layer "F.Cu") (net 44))
 (segment (start 190 92.5) (end 154 92.5) (width 1) (layer "F.Cu") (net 44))
 (segment (start 191 93.5) (end 190 92.5) (width 1) (layer "F.Cu") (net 44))
 (segment (start 195.25 93.5) (end 191 93.5) (width 1) (layer "F.Cu") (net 44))
 (segment (start 211.02 95.9) (end 208.62 93.5) (width 1) (layer "F.Cu") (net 24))
 (segment (start 214.5 95.9) (end 211.02 95.9) (width 1) (layer "F.Cu") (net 24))
 (segment (start 175.5 63.5) (end 164.757 74.243) (width 1) (layer "F.Cu") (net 11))
 (segment (start 164.757 74.243) (end 142.743 74.243) (width 1) (layer "F.Cu") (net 11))
 (segment (start 142.743 74.243) (end 134 65.5) (width 1) (layer "F.Cu") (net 11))
 (segment (start 134 63) (end 134 65.5) (width 1) (layer "F.Cu") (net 11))
 (segment (start 168.978177 75.443) (end 137.021823 75.443) (width 1) (layer "F.Cu") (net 10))
 (segment (start 178 63.5) (end 178 68.5) (width 1) (layer "F.Cu") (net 10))
 (segment (start 171.05 75.45) (end 168.985177 75.45) (width 1) (layer "F.Cu") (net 10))
 (segment (start 129 69.5) (end 129 65.5) (width 1) (layer "F.Cu") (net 10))
 (segment (start 137.021823 75.443) (end 137.014823 75.45) (width 1) (layer "F.Cu") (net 10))
 (segment (start 134.95 75.45) (end 129 69.5) (width 1) (layer "F.Cu") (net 10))
 (segment (start 178 68.5) (end 171.05 75.45) (width 1) (layer "F.Cu") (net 10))
 (segment (start 168.985177 75.45) (end 168.978177 75.443) (width 1) (layer "F.Cu") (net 10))
 (segment (start 137.014823 75.45) (end 134.95 75.45) (width 1) (layer "F.Cu") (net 10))
 (segment (start 129 63) (end 129 65.5) (width 1) (layer "F.Cu") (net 10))
 (segment (start 170.5 65.106396) (end 163.763396 71.843) (width 1) (layer "F.Cu") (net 41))
 (segment (start 152.5 70) (end 151 68.5) (width 1) (layer "F.Cu") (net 41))
 (segment (start 156.843 71.843) (end 155 70) (width 1) (layer "F.Cu") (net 41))
 (segment (start 163.763396 71.843) (end 156.843 71.843) (width 1) (layer "F.Cu") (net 41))
 (segment (start 150.8 68.3) (end 151 68.5) (width 1) (layer "F.Cu") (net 41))
 (segment (start 148 68.3) (end 150.8 68.3) (width 1) (layer "F.Cu") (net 41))
 (segment (start 170.5 63.5) (end 170.5 65.106396) (width 1) (layer "F.Cu") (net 41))
 (segment (start 155 70) (end 152.5 70) (width 1) (layer "F.Cu") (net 41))
 (segment (start 139 63) (end 139 65.5) (width 1) (layer "F.Cu") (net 12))
 (segment (start 146.543 73.043) (end 139 65.5) (width 1) (layer "F.Cu") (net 12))
 (segment (start 173 64.303452) (end 164.260452 73.043) (width 1) (layer "F.Cu") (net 12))
 (segment (start 173 63.5) (end 173 64.303452) (width 1) (layer "F.Cu") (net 12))
 (segment (start 164.260452 73.043) (end 146.543 73.043) (width 1) (layer "F.Cu") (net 12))
 (segment (start 94 116) (end 99 111) (width 1) (layer "B.Cu") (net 4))
 (segment (start 120.5 111) (end 134.5 97) (width 1) (layer "B.Cu") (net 4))
 (segment (start 134.5 97) (end 175 97) (width 1) (layer "B.Cu") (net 4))
 (segment (start 99 111) (end 120.5 111) (width 1) (layer "B.Cu") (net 4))
 (segment (start 175 97) (end 180 102) (width 1) (layer "B.Cu") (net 4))
 (segment (start 119.04 87.04) (end 117 87.04) (width 1) (layer "F.Cu") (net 2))
 (segment (start 118 101) (end 120.5 98.5) (width 1) (layer "F.Cu") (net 2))
 (segment (start 120.5 88.5) (end 119.04 87.04) (width 1) (layer "F.Cu") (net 2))
 (segment (start 120.5 98.5) (end 120.5 88.5) (width 1) (layer "F.Cu") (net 2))
 (segment (start 217.04 119.962081) (end 216.502081 120.5) (width 1) (layer "B.Cu") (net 5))
 (segment (start 217.04 118.76) (end 217.04 119.962081) (width 1) (layer "B.Cu") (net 5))
 (segment (start 184.411522 94.5) (end 112 94.5) (width 1) (layer "B.Cu") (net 5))
 (segment (start 94 69) (end 94 61) (width 1) (layer "B.Cu") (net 5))
 (segment (start 112 94.5) (end 94 76.5) (width 1) (layer "B.Cu") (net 5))
 (segment (start 94 76.5) (end 94 69) (width 1) (layer "B.Cu") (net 5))
 (segment (start 216.502081 120.5) (end 210.411522 120.5) (width 1) (layer "B.Cu") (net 5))
 (segment (start 210.411522 120.5) (end 184.411522 94.5) (width 1) (layer "B.Cu") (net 5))
 (segment (start 144 65.5) (end 146 65.5) (width 1) (layer "F.Cu") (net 13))
 (segment (start 146.5 65.5) (end 146 65.5) (width 1) (layer "F.Cu") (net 13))
 (segment (start 148 67) (end 146.5 65.5) (width 1) (layer "F.Cu") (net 13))
 (segment (start 154.5 65.5) (end 155 66) (width 1) (layer "F.Cu") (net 13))
 (segment (start 146 65.5) (end 154.5 65.5) (width 1) (layer "F.Cu") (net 13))
 (segment (start 144 63) (end 144 65.5) (width 1) (layer "F.Cu") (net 13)))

